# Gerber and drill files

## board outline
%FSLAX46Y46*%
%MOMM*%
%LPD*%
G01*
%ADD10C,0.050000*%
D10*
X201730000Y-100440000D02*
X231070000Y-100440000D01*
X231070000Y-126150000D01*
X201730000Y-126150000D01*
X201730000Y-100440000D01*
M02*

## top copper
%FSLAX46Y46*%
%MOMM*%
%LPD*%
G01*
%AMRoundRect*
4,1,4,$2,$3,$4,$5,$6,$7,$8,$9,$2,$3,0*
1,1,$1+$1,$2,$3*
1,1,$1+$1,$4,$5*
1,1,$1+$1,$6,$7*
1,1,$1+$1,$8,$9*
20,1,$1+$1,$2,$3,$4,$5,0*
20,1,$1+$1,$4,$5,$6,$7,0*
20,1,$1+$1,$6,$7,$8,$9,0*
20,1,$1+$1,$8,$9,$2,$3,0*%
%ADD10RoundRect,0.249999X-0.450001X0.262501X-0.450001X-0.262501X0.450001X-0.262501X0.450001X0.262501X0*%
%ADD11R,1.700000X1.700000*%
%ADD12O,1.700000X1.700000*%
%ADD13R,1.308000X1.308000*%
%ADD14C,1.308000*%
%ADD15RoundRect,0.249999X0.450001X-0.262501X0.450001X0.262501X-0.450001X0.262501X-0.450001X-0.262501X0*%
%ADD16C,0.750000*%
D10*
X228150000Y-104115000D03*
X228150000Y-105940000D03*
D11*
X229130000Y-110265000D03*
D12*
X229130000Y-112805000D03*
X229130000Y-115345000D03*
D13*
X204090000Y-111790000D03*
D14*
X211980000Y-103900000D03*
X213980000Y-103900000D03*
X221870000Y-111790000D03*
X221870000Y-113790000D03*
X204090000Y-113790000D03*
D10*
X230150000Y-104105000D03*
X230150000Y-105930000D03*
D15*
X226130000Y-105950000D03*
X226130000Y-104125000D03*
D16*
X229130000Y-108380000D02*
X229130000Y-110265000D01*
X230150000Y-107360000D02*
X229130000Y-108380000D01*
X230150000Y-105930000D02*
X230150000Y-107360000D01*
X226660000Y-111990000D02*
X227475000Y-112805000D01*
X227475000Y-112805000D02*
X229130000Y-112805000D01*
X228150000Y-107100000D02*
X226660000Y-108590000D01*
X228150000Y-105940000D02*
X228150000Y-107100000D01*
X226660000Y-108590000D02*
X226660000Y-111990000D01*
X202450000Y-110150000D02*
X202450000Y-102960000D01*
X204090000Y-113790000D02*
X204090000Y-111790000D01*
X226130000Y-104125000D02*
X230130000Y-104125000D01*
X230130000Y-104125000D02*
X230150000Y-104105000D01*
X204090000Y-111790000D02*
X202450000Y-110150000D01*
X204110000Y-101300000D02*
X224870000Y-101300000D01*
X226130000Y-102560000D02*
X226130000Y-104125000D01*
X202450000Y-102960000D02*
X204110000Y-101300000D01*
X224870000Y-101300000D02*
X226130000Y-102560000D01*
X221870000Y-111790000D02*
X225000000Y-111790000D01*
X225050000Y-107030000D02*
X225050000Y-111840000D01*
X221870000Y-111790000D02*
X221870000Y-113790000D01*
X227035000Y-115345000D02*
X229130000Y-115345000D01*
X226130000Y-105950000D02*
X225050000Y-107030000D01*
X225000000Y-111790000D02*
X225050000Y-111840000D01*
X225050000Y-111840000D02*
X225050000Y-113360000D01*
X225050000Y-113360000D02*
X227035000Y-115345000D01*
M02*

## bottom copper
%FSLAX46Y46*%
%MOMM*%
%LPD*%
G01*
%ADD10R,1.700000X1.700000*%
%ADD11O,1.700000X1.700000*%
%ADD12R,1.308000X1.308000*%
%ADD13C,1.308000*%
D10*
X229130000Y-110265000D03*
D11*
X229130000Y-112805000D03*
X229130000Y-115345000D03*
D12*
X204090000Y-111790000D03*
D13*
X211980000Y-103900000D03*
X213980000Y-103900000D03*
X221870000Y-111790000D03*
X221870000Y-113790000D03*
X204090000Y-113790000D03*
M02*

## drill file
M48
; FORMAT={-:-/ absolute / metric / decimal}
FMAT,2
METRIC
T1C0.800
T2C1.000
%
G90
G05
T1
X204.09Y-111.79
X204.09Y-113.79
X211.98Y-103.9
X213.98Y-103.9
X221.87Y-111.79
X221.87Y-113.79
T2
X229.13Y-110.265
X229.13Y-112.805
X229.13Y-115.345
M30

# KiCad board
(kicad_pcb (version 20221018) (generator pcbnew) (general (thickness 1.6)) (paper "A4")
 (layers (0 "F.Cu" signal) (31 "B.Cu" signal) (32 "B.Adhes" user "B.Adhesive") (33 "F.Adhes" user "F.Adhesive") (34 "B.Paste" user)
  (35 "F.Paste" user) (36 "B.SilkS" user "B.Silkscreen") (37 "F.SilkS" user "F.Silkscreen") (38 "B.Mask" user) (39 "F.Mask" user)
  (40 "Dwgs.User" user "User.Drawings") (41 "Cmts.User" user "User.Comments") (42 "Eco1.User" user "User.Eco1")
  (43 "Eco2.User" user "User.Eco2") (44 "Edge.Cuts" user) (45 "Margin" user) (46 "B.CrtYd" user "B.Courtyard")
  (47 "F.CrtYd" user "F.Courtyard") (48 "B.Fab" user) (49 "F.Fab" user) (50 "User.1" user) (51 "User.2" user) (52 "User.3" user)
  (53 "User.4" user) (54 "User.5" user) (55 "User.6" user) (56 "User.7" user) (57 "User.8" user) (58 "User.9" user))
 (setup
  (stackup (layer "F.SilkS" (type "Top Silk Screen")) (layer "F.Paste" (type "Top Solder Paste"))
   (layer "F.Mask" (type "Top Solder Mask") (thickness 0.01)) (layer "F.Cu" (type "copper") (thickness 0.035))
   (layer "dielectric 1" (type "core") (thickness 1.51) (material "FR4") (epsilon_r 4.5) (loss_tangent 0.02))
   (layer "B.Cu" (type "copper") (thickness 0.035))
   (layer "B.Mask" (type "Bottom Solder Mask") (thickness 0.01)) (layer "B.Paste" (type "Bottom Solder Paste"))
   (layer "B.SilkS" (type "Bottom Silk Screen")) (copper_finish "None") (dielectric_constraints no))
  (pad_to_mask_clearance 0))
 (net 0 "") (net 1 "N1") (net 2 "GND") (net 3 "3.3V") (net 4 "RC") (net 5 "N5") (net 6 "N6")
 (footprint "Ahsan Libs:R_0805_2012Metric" (layer "F.Cu") (at 228.15 105.0275 -90)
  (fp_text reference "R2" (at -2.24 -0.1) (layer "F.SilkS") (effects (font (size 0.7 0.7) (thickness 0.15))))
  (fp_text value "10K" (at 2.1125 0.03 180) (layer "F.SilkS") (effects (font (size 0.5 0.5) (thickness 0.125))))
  (pad "1" smd roundrect (at -0.9125 0 270) (size 1.025 1.4) (layers "F.Cu" "F.Paste" "F.Mask") (roundrect_rratio 0.2439014634) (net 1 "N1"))
  (pad "2" smd roundrect (at 0.9125 0 270) (size 1.025 1.4) (layers "F.Cu" "F.Paste" "F.Mask") (roundrect_rratio 0.2439014634) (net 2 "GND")))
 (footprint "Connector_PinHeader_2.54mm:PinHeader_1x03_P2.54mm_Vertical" (layer "F.Cu") (at 229.13 110.265)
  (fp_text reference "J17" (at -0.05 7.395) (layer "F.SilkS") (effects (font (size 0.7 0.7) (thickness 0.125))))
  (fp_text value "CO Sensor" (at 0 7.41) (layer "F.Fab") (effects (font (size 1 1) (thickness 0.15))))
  (pad "1" thru_hole rect (at 0 0) (size 1.7 1.7) (drill 1) (layers "*.Cu" "*.Mask") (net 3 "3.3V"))
  (pad "2" thru_hole oval (at 0 2.54) (size 1.7 1.7) (drill 1) (layers "*.Cu" "*.Mask") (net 2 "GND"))
  (pad "3" thru_hole oval (at 0 5.08) (size 1.7 1.7) (drill 1) (layers "*.Cu" "*.Mask") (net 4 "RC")))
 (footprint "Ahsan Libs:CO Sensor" (layer "F.Cu") (at 212.98 112.79 -90)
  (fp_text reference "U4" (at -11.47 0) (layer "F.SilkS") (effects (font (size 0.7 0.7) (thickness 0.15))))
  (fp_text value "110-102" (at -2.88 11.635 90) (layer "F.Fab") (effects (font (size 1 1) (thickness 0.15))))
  (pad "1" thru_hole rect (at -1 8.89 270) (size 1.308 1.308) (drill 0.8) (layers "*.Cu" "*.Mask") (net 1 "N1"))
  (pad "2" thru_hole circle (at -8.89 1 270) (size 1.308 1.308) (drill 0.8) (layers "*.Cu" "*.Mask") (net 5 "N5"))
  (pad "3" thru_hole circle (at -8.89 -1 270) (size 1.308 1.308) (drill 0.8) (layers "*.Cu" "*.Mask") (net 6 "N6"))
  (pad "4" thru_hole circle (at -1 -8.89 270) (size 1.308 1.308) (drill 0.8) (layers "*.Cu" "*.Mask") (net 4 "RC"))
  (pad "5" thru_hole circle (at 1 -8.89 270) (size 1.308 1.308) (drill 0.8) (layers "*.Cu" "*.Mask") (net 4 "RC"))
  (pad "6" thru_hole circle (at 1 8.89 270) (size 1.308 1.308) (drill 0.8) (layers "*.Cu" "*.Mask") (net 1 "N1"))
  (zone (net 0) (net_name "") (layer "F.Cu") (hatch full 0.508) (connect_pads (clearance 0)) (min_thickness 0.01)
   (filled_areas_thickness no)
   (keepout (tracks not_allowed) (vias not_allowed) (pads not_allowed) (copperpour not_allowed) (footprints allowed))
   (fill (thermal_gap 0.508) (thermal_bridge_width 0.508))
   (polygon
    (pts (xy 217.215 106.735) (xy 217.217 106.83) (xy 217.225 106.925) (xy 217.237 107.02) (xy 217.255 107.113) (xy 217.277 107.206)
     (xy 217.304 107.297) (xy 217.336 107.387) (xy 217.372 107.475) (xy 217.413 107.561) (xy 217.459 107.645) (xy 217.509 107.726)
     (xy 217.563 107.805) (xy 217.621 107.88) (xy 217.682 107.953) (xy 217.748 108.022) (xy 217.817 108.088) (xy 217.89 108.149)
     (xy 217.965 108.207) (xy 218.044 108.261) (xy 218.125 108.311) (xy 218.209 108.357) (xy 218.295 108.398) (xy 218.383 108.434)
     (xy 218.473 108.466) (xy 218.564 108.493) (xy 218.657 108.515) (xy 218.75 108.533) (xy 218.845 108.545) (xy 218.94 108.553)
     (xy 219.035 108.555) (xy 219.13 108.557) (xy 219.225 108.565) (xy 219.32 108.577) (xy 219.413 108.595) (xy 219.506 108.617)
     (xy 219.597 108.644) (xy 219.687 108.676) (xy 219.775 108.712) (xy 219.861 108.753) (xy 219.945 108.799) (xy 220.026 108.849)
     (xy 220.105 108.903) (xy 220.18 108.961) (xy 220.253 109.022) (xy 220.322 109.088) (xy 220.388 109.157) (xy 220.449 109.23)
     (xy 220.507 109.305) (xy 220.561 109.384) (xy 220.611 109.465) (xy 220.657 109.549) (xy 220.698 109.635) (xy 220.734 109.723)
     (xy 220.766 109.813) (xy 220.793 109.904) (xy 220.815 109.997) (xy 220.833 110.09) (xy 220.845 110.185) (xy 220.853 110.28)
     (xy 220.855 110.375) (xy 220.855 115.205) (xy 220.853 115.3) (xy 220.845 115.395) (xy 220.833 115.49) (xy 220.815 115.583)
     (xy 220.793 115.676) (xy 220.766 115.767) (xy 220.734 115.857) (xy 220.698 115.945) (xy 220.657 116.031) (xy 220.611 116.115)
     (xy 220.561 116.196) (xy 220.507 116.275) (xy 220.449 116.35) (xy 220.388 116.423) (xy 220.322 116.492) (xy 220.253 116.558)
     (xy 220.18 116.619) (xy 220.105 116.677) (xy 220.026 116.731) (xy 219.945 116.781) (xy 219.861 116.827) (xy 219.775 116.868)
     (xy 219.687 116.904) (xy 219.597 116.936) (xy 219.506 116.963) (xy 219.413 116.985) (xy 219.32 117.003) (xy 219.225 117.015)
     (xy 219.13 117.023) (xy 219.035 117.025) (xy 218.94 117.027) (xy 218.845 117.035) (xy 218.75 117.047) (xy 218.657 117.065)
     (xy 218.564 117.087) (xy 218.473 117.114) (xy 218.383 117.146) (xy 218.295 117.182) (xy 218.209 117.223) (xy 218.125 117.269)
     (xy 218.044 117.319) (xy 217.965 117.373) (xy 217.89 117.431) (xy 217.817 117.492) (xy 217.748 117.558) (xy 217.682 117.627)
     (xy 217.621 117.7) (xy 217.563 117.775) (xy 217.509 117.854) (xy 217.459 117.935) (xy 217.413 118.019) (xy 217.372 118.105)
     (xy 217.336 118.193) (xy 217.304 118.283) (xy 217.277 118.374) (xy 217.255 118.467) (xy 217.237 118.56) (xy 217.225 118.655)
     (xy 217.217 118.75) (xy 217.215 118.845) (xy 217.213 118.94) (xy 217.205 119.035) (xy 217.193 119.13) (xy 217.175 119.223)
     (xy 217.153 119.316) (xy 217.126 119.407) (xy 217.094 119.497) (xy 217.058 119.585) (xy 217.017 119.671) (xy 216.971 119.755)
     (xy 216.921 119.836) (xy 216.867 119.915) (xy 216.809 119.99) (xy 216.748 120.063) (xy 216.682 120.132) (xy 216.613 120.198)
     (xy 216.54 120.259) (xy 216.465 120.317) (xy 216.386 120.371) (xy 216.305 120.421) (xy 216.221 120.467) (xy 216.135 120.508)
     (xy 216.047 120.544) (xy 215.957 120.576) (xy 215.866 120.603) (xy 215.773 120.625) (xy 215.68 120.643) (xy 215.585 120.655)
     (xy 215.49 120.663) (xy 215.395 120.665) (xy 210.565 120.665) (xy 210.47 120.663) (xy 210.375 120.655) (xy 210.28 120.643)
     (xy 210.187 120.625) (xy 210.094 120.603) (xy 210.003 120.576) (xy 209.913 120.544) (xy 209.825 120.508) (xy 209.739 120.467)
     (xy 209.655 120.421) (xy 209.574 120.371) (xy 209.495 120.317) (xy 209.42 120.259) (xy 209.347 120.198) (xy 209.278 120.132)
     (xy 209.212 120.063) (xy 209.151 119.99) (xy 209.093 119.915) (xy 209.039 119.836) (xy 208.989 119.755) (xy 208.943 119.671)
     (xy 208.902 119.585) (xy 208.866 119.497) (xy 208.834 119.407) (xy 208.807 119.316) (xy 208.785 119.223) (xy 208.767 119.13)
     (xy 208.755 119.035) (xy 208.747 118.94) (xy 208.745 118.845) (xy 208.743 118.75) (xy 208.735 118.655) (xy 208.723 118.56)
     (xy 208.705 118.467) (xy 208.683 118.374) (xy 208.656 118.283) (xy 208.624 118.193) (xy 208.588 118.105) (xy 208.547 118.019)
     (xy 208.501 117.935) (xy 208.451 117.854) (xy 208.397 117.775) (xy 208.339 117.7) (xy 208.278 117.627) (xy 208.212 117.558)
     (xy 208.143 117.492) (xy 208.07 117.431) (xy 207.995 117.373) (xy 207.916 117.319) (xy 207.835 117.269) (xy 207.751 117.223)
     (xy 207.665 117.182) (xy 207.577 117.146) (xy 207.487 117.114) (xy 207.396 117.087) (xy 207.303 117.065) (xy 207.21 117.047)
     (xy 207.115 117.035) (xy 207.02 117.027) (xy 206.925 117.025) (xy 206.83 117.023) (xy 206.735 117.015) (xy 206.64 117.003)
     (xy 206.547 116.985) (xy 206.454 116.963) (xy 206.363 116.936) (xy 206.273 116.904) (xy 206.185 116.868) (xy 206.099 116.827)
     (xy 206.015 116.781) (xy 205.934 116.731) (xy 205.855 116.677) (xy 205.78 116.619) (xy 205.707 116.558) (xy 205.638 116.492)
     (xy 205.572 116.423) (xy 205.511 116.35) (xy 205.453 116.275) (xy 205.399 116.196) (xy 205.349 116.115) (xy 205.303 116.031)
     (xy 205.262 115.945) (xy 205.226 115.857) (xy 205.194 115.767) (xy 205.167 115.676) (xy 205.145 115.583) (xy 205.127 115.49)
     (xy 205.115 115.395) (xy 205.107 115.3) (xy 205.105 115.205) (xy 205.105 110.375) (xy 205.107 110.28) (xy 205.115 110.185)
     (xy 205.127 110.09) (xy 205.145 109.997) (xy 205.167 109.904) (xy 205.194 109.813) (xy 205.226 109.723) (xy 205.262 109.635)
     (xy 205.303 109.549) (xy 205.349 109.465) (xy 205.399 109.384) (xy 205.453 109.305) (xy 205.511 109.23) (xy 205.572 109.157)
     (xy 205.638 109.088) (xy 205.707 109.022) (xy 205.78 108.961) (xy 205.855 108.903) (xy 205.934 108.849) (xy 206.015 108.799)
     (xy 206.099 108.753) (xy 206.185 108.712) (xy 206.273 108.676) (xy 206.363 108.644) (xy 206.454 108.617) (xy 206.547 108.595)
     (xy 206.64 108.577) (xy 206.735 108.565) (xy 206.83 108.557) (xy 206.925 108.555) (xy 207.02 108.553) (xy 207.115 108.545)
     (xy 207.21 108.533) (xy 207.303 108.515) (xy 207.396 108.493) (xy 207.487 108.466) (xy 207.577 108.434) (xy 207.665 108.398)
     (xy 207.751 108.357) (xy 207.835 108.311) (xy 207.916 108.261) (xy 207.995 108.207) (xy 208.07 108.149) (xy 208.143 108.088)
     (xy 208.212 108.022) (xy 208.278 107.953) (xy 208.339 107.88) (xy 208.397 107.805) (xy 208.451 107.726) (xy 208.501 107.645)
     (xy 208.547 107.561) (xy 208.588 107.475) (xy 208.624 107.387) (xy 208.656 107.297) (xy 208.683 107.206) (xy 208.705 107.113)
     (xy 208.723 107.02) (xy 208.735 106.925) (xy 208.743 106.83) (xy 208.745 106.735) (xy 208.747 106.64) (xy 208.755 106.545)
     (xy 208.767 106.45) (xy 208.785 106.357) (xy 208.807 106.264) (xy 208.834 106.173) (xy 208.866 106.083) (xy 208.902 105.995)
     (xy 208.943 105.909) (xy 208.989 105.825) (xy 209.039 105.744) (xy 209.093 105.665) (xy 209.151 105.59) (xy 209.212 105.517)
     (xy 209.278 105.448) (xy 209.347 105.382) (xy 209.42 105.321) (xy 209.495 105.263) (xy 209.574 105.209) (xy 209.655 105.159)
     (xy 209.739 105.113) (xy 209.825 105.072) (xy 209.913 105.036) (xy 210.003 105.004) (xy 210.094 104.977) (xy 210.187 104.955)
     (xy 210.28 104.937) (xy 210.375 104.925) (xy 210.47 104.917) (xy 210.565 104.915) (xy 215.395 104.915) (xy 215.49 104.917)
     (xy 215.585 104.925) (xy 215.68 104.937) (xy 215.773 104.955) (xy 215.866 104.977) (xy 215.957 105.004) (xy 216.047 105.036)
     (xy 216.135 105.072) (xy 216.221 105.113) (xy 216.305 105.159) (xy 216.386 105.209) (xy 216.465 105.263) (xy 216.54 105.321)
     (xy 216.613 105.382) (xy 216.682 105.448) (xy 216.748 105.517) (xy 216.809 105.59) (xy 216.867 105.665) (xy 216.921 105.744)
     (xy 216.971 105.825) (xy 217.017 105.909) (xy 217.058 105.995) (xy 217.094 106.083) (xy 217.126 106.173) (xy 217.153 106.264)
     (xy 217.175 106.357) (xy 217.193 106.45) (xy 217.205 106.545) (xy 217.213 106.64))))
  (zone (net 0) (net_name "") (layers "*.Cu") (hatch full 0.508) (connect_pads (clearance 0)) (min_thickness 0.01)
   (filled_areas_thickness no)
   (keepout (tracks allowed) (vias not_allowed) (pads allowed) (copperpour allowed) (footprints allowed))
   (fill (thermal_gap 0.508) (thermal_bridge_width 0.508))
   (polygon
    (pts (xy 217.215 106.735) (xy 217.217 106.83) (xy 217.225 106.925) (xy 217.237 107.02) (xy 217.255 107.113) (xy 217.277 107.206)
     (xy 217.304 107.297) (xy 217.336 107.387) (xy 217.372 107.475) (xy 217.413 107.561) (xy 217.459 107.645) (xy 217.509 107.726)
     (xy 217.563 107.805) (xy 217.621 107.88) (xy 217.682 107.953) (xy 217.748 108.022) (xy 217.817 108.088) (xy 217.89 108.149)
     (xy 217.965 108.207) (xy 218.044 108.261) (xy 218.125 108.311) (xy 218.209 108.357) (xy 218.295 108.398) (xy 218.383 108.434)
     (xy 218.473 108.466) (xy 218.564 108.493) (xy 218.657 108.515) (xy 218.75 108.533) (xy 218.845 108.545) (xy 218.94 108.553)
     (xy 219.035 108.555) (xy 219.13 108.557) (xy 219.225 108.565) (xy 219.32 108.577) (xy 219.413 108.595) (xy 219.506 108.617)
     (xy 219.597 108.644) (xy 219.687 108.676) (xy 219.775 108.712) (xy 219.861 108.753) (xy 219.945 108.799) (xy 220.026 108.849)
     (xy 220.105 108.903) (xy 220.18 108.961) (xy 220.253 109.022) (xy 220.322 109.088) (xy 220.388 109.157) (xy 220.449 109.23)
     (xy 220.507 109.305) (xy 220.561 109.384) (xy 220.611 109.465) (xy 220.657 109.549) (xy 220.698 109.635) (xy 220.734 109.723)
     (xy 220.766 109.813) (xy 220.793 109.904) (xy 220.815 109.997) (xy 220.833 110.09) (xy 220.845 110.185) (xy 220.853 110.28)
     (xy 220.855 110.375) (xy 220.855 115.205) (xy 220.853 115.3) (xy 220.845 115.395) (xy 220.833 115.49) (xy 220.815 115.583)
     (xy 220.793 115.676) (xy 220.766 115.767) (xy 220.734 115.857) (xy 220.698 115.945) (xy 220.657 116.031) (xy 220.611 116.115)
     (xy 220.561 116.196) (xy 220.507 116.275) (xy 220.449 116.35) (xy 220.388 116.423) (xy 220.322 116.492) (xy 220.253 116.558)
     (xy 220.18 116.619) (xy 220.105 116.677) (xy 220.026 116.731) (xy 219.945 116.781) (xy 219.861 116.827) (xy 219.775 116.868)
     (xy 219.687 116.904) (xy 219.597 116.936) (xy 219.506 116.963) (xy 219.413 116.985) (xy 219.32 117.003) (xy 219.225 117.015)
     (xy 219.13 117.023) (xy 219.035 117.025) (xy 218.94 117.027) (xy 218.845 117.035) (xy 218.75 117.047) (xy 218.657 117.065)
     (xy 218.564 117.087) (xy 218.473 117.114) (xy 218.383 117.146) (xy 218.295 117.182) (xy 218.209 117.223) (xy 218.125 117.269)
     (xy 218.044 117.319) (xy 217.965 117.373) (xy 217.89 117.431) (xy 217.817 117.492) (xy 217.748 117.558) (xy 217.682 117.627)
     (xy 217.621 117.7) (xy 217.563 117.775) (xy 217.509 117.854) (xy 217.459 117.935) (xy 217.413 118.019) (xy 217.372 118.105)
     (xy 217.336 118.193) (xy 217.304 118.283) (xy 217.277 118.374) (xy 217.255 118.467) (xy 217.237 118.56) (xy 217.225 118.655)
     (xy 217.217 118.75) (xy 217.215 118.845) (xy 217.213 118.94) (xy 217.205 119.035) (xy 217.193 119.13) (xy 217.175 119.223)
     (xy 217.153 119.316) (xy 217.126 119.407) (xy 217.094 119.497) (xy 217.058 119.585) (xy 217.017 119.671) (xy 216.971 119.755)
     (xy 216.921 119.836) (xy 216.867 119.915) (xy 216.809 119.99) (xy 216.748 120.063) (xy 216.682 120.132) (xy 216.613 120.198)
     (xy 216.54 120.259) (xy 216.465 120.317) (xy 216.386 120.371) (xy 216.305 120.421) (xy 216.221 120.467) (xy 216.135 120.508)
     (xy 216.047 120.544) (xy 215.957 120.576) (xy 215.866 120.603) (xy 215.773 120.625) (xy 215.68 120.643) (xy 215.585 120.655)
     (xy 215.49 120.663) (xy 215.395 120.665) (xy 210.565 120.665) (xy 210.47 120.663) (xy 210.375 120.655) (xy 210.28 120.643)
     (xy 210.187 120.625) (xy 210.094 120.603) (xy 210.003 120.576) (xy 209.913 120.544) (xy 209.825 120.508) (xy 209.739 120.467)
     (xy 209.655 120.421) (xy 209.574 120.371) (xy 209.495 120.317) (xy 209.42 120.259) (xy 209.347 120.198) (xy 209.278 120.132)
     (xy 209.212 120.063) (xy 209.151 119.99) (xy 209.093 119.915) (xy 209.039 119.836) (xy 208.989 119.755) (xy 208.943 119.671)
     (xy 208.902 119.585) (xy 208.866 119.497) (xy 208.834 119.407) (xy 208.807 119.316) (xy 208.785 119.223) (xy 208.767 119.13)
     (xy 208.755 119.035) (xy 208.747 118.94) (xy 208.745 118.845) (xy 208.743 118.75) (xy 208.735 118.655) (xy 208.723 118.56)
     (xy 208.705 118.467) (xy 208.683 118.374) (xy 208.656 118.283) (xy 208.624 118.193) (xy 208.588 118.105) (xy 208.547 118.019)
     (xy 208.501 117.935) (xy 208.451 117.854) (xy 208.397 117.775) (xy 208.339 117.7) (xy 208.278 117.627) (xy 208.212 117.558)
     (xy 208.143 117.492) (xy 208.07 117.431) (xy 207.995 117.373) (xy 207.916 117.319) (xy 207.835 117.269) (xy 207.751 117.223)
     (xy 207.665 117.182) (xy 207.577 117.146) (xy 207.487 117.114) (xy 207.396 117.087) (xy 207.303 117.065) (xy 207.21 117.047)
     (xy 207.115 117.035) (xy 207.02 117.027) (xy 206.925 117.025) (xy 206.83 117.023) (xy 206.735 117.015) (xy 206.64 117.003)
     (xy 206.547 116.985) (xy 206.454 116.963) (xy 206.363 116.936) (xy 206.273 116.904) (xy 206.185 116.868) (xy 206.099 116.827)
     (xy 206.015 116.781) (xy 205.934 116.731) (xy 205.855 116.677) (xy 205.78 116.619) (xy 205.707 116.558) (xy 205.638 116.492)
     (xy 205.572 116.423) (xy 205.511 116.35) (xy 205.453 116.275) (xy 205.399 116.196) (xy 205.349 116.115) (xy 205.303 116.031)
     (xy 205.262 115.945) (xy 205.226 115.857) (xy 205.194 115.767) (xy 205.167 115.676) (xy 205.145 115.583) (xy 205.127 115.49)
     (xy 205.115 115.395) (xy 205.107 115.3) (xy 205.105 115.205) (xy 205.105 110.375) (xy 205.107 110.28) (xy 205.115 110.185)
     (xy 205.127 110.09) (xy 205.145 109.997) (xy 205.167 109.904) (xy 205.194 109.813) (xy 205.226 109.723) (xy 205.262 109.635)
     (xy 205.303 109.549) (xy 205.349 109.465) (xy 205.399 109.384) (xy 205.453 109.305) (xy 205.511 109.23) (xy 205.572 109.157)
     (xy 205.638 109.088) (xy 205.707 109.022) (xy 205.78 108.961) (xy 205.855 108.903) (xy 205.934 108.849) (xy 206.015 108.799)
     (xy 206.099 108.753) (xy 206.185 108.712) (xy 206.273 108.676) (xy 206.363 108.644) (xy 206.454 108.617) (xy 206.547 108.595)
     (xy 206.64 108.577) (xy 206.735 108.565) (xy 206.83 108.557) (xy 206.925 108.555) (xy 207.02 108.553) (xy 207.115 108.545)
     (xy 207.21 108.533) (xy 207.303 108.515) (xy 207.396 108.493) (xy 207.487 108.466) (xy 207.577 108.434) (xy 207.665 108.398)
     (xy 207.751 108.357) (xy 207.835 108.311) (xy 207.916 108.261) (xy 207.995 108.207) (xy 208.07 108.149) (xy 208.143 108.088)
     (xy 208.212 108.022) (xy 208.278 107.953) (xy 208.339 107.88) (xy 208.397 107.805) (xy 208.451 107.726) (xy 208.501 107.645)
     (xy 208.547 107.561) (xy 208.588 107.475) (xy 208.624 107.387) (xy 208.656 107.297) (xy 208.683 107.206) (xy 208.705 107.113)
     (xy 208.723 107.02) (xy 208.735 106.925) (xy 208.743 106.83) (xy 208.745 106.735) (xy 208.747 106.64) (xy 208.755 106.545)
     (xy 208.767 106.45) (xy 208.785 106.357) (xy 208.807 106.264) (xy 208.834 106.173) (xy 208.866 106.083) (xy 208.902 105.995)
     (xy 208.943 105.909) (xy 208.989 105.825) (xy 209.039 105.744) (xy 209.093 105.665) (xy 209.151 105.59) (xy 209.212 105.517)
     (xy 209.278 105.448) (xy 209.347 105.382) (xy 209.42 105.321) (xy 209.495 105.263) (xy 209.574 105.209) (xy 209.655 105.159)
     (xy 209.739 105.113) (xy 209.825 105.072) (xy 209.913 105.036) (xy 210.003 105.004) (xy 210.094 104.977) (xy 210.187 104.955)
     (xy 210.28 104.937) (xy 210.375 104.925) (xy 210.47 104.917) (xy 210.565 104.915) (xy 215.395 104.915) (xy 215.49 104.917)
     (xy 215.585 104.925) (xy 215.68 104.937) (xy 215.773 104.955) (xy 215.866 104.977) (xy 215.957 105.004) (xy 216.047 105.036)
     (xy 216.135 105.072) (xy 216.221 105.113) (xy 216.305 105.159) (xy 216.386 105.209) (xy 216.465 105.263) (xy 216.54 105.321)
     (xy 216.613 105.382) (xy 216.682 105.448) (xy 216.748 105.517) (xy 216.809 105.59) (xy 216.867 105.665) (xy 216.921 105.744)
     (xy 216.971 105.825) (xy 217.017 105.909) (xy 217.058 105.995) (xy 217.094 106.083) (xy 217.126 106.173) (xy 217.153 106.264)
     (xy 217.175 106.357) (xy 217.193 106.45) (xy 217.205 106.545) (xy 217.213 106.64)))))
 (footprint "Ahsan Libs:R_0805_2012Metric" (layer "F.Cu") (at 230.15 105.0175 -90)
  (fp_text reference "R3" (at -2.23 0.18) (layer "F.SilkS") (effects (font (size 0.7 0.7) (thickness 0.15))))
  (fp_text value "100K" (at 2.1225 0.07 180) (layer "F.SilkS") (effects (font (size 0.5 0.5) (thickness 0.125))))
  (pad "1" smd roundrect (at -0.9125 0 270) (size 1.025 1.4) (layers "F.Cu" "F.Paste" "F.Mask") (roundrect_rratio 0.2439014634) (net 1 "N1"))
  (pad "2" smd roundrect (at 0.9125 0 270) (size 1.025 1.4) (layers "F.Cu" "F.Paste" "F.Mask") (roundrect_rratio 0.2439014634)
   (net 3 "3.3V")))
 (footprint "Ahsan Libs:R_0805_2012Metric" (layer "F.Cu") (at 226.13 105.0375 90)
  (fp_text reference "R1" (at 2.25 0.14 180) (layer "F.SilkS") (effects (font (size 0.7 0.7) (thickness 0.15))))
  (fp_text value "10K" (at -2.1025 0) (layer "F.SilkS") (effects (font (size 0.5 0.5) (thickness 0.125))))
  (pad "1" smd roundrect (at -0.9125 0 90) (size 1.025 1.4) (layers "F.Cu" "F.Paste" "F.Mask") (roundrect_rratio 0.2439014634) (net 4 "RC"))
  (pad "2" smd roundrect (at 0.9125 0 90) (size 1.025 1.4) (layers "F.Cu" "F.Paste" "F.Mask") (roundrect_rratio 0.2439014634) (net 1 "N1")))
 (gr_rect (start 201.73 100.44) (end 231.07 126.15) (stroke (width 0.05) (type default)) (fill none) (layer "Edge.Cuts"))
 (segment (start 229.13 108.38) (end 229.13 110.265) (width 0.75) (layer "F.Cu") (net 3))
 (segment (start 230.15 107.36) (end 229.13 108.38) (width 0.75) (layer "F.Cu") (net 3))
 (segment (start 230.15 105.93) (end 230.15 107.36) (width 0.75) (layer "F.Cu") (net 3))
 (segment (start 226.66 111.99) (end 227.475 112.805) (width 0.75) (layer "F.Cu") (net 2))
 (segment (start 227.475 112.805) (end 229.13 112.805) (width 0.75) (layer "F.Cu") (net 2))
 (segment (start 228.15 107.1) (end 226.66 108.59) (width 0.75) (layer "F.Cu") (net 2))
 (segment (start 228.15 105.94) (end 228.15 107.1) (width 0.75) (layer "F.Cu") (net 2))
 (segment (start 226.66 108.59) (end 226.66 111.99) (width 0.75) (layer "F.Cu") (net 2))
 (segment (start 202.45 110.15) (end 202.45 102.96) (width 0.75) (layer "F.Cu") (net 1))
 (segment (start 204.09 113.79) (end 204.09 111.79) (width 0.75) (layer "F.Cu") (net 1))
 (segment (start 226.13 104.125) (end 230.13 104.125) (width 0.75) (layer "F.Cu") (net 1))
 (segment (start 230.13 104.125) (end 230.15 104.105) (width 0.75) (layer "F.Cu") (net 1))
 (segment (start 204.09 111.79) (end 202.45 110.15) (width 0.75) (layer "F.Cu") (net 1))
 (segment (start 204.11 101.3) (end 224.87 101.3) (width 0.75) (layer "F.Cu") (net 1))
 (segment (start 226.13 102.56) (end 226.13 104.125) (width 0.75) (layer "F.Cu") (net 1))
 (segment (start 202.45 102.96) (end 204.11 101.3) (width 0.75) (layer "F.Cu") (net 1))
 (segment (start 224.87 101.3) (end 226.13 102.56) (width 0.75) (layer "F.Cu") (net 1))
 (segment (start 221.87 111.79) (end 225 111.79) (width 0.75) (layer "F.Cu") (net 4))
 (segment (start 225.05 107.03) (end 225.05 111.84) (width 0.75) (layer "F.Cu") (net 4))
 (segment (start 221.87 111.79) (end 221.87 113.79) (width 0.75) (layer "F.Cu") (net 4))
 (segment (start 227.035 115.345) (end 229.13 115.345) (width 0.75) (layer "F.Cu") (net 4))
 (segment (start 226.13 105.95) (end 225.05 107.03) (width 0.75) (layer "F.Cu") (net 4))
 (segment (start 225 111.79) (end 225.05 111.84) (width 0.75) (layer "F.Cu") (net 4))
 (segment (start 225.05 111.84) (end 225.05 113.36) (width 0.75) (layer "F.Cu") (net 4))
 (segment (start 225.05 113.36) (end 227.035 115.345) (width 0.75) (layer "F.Cu") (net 4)))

